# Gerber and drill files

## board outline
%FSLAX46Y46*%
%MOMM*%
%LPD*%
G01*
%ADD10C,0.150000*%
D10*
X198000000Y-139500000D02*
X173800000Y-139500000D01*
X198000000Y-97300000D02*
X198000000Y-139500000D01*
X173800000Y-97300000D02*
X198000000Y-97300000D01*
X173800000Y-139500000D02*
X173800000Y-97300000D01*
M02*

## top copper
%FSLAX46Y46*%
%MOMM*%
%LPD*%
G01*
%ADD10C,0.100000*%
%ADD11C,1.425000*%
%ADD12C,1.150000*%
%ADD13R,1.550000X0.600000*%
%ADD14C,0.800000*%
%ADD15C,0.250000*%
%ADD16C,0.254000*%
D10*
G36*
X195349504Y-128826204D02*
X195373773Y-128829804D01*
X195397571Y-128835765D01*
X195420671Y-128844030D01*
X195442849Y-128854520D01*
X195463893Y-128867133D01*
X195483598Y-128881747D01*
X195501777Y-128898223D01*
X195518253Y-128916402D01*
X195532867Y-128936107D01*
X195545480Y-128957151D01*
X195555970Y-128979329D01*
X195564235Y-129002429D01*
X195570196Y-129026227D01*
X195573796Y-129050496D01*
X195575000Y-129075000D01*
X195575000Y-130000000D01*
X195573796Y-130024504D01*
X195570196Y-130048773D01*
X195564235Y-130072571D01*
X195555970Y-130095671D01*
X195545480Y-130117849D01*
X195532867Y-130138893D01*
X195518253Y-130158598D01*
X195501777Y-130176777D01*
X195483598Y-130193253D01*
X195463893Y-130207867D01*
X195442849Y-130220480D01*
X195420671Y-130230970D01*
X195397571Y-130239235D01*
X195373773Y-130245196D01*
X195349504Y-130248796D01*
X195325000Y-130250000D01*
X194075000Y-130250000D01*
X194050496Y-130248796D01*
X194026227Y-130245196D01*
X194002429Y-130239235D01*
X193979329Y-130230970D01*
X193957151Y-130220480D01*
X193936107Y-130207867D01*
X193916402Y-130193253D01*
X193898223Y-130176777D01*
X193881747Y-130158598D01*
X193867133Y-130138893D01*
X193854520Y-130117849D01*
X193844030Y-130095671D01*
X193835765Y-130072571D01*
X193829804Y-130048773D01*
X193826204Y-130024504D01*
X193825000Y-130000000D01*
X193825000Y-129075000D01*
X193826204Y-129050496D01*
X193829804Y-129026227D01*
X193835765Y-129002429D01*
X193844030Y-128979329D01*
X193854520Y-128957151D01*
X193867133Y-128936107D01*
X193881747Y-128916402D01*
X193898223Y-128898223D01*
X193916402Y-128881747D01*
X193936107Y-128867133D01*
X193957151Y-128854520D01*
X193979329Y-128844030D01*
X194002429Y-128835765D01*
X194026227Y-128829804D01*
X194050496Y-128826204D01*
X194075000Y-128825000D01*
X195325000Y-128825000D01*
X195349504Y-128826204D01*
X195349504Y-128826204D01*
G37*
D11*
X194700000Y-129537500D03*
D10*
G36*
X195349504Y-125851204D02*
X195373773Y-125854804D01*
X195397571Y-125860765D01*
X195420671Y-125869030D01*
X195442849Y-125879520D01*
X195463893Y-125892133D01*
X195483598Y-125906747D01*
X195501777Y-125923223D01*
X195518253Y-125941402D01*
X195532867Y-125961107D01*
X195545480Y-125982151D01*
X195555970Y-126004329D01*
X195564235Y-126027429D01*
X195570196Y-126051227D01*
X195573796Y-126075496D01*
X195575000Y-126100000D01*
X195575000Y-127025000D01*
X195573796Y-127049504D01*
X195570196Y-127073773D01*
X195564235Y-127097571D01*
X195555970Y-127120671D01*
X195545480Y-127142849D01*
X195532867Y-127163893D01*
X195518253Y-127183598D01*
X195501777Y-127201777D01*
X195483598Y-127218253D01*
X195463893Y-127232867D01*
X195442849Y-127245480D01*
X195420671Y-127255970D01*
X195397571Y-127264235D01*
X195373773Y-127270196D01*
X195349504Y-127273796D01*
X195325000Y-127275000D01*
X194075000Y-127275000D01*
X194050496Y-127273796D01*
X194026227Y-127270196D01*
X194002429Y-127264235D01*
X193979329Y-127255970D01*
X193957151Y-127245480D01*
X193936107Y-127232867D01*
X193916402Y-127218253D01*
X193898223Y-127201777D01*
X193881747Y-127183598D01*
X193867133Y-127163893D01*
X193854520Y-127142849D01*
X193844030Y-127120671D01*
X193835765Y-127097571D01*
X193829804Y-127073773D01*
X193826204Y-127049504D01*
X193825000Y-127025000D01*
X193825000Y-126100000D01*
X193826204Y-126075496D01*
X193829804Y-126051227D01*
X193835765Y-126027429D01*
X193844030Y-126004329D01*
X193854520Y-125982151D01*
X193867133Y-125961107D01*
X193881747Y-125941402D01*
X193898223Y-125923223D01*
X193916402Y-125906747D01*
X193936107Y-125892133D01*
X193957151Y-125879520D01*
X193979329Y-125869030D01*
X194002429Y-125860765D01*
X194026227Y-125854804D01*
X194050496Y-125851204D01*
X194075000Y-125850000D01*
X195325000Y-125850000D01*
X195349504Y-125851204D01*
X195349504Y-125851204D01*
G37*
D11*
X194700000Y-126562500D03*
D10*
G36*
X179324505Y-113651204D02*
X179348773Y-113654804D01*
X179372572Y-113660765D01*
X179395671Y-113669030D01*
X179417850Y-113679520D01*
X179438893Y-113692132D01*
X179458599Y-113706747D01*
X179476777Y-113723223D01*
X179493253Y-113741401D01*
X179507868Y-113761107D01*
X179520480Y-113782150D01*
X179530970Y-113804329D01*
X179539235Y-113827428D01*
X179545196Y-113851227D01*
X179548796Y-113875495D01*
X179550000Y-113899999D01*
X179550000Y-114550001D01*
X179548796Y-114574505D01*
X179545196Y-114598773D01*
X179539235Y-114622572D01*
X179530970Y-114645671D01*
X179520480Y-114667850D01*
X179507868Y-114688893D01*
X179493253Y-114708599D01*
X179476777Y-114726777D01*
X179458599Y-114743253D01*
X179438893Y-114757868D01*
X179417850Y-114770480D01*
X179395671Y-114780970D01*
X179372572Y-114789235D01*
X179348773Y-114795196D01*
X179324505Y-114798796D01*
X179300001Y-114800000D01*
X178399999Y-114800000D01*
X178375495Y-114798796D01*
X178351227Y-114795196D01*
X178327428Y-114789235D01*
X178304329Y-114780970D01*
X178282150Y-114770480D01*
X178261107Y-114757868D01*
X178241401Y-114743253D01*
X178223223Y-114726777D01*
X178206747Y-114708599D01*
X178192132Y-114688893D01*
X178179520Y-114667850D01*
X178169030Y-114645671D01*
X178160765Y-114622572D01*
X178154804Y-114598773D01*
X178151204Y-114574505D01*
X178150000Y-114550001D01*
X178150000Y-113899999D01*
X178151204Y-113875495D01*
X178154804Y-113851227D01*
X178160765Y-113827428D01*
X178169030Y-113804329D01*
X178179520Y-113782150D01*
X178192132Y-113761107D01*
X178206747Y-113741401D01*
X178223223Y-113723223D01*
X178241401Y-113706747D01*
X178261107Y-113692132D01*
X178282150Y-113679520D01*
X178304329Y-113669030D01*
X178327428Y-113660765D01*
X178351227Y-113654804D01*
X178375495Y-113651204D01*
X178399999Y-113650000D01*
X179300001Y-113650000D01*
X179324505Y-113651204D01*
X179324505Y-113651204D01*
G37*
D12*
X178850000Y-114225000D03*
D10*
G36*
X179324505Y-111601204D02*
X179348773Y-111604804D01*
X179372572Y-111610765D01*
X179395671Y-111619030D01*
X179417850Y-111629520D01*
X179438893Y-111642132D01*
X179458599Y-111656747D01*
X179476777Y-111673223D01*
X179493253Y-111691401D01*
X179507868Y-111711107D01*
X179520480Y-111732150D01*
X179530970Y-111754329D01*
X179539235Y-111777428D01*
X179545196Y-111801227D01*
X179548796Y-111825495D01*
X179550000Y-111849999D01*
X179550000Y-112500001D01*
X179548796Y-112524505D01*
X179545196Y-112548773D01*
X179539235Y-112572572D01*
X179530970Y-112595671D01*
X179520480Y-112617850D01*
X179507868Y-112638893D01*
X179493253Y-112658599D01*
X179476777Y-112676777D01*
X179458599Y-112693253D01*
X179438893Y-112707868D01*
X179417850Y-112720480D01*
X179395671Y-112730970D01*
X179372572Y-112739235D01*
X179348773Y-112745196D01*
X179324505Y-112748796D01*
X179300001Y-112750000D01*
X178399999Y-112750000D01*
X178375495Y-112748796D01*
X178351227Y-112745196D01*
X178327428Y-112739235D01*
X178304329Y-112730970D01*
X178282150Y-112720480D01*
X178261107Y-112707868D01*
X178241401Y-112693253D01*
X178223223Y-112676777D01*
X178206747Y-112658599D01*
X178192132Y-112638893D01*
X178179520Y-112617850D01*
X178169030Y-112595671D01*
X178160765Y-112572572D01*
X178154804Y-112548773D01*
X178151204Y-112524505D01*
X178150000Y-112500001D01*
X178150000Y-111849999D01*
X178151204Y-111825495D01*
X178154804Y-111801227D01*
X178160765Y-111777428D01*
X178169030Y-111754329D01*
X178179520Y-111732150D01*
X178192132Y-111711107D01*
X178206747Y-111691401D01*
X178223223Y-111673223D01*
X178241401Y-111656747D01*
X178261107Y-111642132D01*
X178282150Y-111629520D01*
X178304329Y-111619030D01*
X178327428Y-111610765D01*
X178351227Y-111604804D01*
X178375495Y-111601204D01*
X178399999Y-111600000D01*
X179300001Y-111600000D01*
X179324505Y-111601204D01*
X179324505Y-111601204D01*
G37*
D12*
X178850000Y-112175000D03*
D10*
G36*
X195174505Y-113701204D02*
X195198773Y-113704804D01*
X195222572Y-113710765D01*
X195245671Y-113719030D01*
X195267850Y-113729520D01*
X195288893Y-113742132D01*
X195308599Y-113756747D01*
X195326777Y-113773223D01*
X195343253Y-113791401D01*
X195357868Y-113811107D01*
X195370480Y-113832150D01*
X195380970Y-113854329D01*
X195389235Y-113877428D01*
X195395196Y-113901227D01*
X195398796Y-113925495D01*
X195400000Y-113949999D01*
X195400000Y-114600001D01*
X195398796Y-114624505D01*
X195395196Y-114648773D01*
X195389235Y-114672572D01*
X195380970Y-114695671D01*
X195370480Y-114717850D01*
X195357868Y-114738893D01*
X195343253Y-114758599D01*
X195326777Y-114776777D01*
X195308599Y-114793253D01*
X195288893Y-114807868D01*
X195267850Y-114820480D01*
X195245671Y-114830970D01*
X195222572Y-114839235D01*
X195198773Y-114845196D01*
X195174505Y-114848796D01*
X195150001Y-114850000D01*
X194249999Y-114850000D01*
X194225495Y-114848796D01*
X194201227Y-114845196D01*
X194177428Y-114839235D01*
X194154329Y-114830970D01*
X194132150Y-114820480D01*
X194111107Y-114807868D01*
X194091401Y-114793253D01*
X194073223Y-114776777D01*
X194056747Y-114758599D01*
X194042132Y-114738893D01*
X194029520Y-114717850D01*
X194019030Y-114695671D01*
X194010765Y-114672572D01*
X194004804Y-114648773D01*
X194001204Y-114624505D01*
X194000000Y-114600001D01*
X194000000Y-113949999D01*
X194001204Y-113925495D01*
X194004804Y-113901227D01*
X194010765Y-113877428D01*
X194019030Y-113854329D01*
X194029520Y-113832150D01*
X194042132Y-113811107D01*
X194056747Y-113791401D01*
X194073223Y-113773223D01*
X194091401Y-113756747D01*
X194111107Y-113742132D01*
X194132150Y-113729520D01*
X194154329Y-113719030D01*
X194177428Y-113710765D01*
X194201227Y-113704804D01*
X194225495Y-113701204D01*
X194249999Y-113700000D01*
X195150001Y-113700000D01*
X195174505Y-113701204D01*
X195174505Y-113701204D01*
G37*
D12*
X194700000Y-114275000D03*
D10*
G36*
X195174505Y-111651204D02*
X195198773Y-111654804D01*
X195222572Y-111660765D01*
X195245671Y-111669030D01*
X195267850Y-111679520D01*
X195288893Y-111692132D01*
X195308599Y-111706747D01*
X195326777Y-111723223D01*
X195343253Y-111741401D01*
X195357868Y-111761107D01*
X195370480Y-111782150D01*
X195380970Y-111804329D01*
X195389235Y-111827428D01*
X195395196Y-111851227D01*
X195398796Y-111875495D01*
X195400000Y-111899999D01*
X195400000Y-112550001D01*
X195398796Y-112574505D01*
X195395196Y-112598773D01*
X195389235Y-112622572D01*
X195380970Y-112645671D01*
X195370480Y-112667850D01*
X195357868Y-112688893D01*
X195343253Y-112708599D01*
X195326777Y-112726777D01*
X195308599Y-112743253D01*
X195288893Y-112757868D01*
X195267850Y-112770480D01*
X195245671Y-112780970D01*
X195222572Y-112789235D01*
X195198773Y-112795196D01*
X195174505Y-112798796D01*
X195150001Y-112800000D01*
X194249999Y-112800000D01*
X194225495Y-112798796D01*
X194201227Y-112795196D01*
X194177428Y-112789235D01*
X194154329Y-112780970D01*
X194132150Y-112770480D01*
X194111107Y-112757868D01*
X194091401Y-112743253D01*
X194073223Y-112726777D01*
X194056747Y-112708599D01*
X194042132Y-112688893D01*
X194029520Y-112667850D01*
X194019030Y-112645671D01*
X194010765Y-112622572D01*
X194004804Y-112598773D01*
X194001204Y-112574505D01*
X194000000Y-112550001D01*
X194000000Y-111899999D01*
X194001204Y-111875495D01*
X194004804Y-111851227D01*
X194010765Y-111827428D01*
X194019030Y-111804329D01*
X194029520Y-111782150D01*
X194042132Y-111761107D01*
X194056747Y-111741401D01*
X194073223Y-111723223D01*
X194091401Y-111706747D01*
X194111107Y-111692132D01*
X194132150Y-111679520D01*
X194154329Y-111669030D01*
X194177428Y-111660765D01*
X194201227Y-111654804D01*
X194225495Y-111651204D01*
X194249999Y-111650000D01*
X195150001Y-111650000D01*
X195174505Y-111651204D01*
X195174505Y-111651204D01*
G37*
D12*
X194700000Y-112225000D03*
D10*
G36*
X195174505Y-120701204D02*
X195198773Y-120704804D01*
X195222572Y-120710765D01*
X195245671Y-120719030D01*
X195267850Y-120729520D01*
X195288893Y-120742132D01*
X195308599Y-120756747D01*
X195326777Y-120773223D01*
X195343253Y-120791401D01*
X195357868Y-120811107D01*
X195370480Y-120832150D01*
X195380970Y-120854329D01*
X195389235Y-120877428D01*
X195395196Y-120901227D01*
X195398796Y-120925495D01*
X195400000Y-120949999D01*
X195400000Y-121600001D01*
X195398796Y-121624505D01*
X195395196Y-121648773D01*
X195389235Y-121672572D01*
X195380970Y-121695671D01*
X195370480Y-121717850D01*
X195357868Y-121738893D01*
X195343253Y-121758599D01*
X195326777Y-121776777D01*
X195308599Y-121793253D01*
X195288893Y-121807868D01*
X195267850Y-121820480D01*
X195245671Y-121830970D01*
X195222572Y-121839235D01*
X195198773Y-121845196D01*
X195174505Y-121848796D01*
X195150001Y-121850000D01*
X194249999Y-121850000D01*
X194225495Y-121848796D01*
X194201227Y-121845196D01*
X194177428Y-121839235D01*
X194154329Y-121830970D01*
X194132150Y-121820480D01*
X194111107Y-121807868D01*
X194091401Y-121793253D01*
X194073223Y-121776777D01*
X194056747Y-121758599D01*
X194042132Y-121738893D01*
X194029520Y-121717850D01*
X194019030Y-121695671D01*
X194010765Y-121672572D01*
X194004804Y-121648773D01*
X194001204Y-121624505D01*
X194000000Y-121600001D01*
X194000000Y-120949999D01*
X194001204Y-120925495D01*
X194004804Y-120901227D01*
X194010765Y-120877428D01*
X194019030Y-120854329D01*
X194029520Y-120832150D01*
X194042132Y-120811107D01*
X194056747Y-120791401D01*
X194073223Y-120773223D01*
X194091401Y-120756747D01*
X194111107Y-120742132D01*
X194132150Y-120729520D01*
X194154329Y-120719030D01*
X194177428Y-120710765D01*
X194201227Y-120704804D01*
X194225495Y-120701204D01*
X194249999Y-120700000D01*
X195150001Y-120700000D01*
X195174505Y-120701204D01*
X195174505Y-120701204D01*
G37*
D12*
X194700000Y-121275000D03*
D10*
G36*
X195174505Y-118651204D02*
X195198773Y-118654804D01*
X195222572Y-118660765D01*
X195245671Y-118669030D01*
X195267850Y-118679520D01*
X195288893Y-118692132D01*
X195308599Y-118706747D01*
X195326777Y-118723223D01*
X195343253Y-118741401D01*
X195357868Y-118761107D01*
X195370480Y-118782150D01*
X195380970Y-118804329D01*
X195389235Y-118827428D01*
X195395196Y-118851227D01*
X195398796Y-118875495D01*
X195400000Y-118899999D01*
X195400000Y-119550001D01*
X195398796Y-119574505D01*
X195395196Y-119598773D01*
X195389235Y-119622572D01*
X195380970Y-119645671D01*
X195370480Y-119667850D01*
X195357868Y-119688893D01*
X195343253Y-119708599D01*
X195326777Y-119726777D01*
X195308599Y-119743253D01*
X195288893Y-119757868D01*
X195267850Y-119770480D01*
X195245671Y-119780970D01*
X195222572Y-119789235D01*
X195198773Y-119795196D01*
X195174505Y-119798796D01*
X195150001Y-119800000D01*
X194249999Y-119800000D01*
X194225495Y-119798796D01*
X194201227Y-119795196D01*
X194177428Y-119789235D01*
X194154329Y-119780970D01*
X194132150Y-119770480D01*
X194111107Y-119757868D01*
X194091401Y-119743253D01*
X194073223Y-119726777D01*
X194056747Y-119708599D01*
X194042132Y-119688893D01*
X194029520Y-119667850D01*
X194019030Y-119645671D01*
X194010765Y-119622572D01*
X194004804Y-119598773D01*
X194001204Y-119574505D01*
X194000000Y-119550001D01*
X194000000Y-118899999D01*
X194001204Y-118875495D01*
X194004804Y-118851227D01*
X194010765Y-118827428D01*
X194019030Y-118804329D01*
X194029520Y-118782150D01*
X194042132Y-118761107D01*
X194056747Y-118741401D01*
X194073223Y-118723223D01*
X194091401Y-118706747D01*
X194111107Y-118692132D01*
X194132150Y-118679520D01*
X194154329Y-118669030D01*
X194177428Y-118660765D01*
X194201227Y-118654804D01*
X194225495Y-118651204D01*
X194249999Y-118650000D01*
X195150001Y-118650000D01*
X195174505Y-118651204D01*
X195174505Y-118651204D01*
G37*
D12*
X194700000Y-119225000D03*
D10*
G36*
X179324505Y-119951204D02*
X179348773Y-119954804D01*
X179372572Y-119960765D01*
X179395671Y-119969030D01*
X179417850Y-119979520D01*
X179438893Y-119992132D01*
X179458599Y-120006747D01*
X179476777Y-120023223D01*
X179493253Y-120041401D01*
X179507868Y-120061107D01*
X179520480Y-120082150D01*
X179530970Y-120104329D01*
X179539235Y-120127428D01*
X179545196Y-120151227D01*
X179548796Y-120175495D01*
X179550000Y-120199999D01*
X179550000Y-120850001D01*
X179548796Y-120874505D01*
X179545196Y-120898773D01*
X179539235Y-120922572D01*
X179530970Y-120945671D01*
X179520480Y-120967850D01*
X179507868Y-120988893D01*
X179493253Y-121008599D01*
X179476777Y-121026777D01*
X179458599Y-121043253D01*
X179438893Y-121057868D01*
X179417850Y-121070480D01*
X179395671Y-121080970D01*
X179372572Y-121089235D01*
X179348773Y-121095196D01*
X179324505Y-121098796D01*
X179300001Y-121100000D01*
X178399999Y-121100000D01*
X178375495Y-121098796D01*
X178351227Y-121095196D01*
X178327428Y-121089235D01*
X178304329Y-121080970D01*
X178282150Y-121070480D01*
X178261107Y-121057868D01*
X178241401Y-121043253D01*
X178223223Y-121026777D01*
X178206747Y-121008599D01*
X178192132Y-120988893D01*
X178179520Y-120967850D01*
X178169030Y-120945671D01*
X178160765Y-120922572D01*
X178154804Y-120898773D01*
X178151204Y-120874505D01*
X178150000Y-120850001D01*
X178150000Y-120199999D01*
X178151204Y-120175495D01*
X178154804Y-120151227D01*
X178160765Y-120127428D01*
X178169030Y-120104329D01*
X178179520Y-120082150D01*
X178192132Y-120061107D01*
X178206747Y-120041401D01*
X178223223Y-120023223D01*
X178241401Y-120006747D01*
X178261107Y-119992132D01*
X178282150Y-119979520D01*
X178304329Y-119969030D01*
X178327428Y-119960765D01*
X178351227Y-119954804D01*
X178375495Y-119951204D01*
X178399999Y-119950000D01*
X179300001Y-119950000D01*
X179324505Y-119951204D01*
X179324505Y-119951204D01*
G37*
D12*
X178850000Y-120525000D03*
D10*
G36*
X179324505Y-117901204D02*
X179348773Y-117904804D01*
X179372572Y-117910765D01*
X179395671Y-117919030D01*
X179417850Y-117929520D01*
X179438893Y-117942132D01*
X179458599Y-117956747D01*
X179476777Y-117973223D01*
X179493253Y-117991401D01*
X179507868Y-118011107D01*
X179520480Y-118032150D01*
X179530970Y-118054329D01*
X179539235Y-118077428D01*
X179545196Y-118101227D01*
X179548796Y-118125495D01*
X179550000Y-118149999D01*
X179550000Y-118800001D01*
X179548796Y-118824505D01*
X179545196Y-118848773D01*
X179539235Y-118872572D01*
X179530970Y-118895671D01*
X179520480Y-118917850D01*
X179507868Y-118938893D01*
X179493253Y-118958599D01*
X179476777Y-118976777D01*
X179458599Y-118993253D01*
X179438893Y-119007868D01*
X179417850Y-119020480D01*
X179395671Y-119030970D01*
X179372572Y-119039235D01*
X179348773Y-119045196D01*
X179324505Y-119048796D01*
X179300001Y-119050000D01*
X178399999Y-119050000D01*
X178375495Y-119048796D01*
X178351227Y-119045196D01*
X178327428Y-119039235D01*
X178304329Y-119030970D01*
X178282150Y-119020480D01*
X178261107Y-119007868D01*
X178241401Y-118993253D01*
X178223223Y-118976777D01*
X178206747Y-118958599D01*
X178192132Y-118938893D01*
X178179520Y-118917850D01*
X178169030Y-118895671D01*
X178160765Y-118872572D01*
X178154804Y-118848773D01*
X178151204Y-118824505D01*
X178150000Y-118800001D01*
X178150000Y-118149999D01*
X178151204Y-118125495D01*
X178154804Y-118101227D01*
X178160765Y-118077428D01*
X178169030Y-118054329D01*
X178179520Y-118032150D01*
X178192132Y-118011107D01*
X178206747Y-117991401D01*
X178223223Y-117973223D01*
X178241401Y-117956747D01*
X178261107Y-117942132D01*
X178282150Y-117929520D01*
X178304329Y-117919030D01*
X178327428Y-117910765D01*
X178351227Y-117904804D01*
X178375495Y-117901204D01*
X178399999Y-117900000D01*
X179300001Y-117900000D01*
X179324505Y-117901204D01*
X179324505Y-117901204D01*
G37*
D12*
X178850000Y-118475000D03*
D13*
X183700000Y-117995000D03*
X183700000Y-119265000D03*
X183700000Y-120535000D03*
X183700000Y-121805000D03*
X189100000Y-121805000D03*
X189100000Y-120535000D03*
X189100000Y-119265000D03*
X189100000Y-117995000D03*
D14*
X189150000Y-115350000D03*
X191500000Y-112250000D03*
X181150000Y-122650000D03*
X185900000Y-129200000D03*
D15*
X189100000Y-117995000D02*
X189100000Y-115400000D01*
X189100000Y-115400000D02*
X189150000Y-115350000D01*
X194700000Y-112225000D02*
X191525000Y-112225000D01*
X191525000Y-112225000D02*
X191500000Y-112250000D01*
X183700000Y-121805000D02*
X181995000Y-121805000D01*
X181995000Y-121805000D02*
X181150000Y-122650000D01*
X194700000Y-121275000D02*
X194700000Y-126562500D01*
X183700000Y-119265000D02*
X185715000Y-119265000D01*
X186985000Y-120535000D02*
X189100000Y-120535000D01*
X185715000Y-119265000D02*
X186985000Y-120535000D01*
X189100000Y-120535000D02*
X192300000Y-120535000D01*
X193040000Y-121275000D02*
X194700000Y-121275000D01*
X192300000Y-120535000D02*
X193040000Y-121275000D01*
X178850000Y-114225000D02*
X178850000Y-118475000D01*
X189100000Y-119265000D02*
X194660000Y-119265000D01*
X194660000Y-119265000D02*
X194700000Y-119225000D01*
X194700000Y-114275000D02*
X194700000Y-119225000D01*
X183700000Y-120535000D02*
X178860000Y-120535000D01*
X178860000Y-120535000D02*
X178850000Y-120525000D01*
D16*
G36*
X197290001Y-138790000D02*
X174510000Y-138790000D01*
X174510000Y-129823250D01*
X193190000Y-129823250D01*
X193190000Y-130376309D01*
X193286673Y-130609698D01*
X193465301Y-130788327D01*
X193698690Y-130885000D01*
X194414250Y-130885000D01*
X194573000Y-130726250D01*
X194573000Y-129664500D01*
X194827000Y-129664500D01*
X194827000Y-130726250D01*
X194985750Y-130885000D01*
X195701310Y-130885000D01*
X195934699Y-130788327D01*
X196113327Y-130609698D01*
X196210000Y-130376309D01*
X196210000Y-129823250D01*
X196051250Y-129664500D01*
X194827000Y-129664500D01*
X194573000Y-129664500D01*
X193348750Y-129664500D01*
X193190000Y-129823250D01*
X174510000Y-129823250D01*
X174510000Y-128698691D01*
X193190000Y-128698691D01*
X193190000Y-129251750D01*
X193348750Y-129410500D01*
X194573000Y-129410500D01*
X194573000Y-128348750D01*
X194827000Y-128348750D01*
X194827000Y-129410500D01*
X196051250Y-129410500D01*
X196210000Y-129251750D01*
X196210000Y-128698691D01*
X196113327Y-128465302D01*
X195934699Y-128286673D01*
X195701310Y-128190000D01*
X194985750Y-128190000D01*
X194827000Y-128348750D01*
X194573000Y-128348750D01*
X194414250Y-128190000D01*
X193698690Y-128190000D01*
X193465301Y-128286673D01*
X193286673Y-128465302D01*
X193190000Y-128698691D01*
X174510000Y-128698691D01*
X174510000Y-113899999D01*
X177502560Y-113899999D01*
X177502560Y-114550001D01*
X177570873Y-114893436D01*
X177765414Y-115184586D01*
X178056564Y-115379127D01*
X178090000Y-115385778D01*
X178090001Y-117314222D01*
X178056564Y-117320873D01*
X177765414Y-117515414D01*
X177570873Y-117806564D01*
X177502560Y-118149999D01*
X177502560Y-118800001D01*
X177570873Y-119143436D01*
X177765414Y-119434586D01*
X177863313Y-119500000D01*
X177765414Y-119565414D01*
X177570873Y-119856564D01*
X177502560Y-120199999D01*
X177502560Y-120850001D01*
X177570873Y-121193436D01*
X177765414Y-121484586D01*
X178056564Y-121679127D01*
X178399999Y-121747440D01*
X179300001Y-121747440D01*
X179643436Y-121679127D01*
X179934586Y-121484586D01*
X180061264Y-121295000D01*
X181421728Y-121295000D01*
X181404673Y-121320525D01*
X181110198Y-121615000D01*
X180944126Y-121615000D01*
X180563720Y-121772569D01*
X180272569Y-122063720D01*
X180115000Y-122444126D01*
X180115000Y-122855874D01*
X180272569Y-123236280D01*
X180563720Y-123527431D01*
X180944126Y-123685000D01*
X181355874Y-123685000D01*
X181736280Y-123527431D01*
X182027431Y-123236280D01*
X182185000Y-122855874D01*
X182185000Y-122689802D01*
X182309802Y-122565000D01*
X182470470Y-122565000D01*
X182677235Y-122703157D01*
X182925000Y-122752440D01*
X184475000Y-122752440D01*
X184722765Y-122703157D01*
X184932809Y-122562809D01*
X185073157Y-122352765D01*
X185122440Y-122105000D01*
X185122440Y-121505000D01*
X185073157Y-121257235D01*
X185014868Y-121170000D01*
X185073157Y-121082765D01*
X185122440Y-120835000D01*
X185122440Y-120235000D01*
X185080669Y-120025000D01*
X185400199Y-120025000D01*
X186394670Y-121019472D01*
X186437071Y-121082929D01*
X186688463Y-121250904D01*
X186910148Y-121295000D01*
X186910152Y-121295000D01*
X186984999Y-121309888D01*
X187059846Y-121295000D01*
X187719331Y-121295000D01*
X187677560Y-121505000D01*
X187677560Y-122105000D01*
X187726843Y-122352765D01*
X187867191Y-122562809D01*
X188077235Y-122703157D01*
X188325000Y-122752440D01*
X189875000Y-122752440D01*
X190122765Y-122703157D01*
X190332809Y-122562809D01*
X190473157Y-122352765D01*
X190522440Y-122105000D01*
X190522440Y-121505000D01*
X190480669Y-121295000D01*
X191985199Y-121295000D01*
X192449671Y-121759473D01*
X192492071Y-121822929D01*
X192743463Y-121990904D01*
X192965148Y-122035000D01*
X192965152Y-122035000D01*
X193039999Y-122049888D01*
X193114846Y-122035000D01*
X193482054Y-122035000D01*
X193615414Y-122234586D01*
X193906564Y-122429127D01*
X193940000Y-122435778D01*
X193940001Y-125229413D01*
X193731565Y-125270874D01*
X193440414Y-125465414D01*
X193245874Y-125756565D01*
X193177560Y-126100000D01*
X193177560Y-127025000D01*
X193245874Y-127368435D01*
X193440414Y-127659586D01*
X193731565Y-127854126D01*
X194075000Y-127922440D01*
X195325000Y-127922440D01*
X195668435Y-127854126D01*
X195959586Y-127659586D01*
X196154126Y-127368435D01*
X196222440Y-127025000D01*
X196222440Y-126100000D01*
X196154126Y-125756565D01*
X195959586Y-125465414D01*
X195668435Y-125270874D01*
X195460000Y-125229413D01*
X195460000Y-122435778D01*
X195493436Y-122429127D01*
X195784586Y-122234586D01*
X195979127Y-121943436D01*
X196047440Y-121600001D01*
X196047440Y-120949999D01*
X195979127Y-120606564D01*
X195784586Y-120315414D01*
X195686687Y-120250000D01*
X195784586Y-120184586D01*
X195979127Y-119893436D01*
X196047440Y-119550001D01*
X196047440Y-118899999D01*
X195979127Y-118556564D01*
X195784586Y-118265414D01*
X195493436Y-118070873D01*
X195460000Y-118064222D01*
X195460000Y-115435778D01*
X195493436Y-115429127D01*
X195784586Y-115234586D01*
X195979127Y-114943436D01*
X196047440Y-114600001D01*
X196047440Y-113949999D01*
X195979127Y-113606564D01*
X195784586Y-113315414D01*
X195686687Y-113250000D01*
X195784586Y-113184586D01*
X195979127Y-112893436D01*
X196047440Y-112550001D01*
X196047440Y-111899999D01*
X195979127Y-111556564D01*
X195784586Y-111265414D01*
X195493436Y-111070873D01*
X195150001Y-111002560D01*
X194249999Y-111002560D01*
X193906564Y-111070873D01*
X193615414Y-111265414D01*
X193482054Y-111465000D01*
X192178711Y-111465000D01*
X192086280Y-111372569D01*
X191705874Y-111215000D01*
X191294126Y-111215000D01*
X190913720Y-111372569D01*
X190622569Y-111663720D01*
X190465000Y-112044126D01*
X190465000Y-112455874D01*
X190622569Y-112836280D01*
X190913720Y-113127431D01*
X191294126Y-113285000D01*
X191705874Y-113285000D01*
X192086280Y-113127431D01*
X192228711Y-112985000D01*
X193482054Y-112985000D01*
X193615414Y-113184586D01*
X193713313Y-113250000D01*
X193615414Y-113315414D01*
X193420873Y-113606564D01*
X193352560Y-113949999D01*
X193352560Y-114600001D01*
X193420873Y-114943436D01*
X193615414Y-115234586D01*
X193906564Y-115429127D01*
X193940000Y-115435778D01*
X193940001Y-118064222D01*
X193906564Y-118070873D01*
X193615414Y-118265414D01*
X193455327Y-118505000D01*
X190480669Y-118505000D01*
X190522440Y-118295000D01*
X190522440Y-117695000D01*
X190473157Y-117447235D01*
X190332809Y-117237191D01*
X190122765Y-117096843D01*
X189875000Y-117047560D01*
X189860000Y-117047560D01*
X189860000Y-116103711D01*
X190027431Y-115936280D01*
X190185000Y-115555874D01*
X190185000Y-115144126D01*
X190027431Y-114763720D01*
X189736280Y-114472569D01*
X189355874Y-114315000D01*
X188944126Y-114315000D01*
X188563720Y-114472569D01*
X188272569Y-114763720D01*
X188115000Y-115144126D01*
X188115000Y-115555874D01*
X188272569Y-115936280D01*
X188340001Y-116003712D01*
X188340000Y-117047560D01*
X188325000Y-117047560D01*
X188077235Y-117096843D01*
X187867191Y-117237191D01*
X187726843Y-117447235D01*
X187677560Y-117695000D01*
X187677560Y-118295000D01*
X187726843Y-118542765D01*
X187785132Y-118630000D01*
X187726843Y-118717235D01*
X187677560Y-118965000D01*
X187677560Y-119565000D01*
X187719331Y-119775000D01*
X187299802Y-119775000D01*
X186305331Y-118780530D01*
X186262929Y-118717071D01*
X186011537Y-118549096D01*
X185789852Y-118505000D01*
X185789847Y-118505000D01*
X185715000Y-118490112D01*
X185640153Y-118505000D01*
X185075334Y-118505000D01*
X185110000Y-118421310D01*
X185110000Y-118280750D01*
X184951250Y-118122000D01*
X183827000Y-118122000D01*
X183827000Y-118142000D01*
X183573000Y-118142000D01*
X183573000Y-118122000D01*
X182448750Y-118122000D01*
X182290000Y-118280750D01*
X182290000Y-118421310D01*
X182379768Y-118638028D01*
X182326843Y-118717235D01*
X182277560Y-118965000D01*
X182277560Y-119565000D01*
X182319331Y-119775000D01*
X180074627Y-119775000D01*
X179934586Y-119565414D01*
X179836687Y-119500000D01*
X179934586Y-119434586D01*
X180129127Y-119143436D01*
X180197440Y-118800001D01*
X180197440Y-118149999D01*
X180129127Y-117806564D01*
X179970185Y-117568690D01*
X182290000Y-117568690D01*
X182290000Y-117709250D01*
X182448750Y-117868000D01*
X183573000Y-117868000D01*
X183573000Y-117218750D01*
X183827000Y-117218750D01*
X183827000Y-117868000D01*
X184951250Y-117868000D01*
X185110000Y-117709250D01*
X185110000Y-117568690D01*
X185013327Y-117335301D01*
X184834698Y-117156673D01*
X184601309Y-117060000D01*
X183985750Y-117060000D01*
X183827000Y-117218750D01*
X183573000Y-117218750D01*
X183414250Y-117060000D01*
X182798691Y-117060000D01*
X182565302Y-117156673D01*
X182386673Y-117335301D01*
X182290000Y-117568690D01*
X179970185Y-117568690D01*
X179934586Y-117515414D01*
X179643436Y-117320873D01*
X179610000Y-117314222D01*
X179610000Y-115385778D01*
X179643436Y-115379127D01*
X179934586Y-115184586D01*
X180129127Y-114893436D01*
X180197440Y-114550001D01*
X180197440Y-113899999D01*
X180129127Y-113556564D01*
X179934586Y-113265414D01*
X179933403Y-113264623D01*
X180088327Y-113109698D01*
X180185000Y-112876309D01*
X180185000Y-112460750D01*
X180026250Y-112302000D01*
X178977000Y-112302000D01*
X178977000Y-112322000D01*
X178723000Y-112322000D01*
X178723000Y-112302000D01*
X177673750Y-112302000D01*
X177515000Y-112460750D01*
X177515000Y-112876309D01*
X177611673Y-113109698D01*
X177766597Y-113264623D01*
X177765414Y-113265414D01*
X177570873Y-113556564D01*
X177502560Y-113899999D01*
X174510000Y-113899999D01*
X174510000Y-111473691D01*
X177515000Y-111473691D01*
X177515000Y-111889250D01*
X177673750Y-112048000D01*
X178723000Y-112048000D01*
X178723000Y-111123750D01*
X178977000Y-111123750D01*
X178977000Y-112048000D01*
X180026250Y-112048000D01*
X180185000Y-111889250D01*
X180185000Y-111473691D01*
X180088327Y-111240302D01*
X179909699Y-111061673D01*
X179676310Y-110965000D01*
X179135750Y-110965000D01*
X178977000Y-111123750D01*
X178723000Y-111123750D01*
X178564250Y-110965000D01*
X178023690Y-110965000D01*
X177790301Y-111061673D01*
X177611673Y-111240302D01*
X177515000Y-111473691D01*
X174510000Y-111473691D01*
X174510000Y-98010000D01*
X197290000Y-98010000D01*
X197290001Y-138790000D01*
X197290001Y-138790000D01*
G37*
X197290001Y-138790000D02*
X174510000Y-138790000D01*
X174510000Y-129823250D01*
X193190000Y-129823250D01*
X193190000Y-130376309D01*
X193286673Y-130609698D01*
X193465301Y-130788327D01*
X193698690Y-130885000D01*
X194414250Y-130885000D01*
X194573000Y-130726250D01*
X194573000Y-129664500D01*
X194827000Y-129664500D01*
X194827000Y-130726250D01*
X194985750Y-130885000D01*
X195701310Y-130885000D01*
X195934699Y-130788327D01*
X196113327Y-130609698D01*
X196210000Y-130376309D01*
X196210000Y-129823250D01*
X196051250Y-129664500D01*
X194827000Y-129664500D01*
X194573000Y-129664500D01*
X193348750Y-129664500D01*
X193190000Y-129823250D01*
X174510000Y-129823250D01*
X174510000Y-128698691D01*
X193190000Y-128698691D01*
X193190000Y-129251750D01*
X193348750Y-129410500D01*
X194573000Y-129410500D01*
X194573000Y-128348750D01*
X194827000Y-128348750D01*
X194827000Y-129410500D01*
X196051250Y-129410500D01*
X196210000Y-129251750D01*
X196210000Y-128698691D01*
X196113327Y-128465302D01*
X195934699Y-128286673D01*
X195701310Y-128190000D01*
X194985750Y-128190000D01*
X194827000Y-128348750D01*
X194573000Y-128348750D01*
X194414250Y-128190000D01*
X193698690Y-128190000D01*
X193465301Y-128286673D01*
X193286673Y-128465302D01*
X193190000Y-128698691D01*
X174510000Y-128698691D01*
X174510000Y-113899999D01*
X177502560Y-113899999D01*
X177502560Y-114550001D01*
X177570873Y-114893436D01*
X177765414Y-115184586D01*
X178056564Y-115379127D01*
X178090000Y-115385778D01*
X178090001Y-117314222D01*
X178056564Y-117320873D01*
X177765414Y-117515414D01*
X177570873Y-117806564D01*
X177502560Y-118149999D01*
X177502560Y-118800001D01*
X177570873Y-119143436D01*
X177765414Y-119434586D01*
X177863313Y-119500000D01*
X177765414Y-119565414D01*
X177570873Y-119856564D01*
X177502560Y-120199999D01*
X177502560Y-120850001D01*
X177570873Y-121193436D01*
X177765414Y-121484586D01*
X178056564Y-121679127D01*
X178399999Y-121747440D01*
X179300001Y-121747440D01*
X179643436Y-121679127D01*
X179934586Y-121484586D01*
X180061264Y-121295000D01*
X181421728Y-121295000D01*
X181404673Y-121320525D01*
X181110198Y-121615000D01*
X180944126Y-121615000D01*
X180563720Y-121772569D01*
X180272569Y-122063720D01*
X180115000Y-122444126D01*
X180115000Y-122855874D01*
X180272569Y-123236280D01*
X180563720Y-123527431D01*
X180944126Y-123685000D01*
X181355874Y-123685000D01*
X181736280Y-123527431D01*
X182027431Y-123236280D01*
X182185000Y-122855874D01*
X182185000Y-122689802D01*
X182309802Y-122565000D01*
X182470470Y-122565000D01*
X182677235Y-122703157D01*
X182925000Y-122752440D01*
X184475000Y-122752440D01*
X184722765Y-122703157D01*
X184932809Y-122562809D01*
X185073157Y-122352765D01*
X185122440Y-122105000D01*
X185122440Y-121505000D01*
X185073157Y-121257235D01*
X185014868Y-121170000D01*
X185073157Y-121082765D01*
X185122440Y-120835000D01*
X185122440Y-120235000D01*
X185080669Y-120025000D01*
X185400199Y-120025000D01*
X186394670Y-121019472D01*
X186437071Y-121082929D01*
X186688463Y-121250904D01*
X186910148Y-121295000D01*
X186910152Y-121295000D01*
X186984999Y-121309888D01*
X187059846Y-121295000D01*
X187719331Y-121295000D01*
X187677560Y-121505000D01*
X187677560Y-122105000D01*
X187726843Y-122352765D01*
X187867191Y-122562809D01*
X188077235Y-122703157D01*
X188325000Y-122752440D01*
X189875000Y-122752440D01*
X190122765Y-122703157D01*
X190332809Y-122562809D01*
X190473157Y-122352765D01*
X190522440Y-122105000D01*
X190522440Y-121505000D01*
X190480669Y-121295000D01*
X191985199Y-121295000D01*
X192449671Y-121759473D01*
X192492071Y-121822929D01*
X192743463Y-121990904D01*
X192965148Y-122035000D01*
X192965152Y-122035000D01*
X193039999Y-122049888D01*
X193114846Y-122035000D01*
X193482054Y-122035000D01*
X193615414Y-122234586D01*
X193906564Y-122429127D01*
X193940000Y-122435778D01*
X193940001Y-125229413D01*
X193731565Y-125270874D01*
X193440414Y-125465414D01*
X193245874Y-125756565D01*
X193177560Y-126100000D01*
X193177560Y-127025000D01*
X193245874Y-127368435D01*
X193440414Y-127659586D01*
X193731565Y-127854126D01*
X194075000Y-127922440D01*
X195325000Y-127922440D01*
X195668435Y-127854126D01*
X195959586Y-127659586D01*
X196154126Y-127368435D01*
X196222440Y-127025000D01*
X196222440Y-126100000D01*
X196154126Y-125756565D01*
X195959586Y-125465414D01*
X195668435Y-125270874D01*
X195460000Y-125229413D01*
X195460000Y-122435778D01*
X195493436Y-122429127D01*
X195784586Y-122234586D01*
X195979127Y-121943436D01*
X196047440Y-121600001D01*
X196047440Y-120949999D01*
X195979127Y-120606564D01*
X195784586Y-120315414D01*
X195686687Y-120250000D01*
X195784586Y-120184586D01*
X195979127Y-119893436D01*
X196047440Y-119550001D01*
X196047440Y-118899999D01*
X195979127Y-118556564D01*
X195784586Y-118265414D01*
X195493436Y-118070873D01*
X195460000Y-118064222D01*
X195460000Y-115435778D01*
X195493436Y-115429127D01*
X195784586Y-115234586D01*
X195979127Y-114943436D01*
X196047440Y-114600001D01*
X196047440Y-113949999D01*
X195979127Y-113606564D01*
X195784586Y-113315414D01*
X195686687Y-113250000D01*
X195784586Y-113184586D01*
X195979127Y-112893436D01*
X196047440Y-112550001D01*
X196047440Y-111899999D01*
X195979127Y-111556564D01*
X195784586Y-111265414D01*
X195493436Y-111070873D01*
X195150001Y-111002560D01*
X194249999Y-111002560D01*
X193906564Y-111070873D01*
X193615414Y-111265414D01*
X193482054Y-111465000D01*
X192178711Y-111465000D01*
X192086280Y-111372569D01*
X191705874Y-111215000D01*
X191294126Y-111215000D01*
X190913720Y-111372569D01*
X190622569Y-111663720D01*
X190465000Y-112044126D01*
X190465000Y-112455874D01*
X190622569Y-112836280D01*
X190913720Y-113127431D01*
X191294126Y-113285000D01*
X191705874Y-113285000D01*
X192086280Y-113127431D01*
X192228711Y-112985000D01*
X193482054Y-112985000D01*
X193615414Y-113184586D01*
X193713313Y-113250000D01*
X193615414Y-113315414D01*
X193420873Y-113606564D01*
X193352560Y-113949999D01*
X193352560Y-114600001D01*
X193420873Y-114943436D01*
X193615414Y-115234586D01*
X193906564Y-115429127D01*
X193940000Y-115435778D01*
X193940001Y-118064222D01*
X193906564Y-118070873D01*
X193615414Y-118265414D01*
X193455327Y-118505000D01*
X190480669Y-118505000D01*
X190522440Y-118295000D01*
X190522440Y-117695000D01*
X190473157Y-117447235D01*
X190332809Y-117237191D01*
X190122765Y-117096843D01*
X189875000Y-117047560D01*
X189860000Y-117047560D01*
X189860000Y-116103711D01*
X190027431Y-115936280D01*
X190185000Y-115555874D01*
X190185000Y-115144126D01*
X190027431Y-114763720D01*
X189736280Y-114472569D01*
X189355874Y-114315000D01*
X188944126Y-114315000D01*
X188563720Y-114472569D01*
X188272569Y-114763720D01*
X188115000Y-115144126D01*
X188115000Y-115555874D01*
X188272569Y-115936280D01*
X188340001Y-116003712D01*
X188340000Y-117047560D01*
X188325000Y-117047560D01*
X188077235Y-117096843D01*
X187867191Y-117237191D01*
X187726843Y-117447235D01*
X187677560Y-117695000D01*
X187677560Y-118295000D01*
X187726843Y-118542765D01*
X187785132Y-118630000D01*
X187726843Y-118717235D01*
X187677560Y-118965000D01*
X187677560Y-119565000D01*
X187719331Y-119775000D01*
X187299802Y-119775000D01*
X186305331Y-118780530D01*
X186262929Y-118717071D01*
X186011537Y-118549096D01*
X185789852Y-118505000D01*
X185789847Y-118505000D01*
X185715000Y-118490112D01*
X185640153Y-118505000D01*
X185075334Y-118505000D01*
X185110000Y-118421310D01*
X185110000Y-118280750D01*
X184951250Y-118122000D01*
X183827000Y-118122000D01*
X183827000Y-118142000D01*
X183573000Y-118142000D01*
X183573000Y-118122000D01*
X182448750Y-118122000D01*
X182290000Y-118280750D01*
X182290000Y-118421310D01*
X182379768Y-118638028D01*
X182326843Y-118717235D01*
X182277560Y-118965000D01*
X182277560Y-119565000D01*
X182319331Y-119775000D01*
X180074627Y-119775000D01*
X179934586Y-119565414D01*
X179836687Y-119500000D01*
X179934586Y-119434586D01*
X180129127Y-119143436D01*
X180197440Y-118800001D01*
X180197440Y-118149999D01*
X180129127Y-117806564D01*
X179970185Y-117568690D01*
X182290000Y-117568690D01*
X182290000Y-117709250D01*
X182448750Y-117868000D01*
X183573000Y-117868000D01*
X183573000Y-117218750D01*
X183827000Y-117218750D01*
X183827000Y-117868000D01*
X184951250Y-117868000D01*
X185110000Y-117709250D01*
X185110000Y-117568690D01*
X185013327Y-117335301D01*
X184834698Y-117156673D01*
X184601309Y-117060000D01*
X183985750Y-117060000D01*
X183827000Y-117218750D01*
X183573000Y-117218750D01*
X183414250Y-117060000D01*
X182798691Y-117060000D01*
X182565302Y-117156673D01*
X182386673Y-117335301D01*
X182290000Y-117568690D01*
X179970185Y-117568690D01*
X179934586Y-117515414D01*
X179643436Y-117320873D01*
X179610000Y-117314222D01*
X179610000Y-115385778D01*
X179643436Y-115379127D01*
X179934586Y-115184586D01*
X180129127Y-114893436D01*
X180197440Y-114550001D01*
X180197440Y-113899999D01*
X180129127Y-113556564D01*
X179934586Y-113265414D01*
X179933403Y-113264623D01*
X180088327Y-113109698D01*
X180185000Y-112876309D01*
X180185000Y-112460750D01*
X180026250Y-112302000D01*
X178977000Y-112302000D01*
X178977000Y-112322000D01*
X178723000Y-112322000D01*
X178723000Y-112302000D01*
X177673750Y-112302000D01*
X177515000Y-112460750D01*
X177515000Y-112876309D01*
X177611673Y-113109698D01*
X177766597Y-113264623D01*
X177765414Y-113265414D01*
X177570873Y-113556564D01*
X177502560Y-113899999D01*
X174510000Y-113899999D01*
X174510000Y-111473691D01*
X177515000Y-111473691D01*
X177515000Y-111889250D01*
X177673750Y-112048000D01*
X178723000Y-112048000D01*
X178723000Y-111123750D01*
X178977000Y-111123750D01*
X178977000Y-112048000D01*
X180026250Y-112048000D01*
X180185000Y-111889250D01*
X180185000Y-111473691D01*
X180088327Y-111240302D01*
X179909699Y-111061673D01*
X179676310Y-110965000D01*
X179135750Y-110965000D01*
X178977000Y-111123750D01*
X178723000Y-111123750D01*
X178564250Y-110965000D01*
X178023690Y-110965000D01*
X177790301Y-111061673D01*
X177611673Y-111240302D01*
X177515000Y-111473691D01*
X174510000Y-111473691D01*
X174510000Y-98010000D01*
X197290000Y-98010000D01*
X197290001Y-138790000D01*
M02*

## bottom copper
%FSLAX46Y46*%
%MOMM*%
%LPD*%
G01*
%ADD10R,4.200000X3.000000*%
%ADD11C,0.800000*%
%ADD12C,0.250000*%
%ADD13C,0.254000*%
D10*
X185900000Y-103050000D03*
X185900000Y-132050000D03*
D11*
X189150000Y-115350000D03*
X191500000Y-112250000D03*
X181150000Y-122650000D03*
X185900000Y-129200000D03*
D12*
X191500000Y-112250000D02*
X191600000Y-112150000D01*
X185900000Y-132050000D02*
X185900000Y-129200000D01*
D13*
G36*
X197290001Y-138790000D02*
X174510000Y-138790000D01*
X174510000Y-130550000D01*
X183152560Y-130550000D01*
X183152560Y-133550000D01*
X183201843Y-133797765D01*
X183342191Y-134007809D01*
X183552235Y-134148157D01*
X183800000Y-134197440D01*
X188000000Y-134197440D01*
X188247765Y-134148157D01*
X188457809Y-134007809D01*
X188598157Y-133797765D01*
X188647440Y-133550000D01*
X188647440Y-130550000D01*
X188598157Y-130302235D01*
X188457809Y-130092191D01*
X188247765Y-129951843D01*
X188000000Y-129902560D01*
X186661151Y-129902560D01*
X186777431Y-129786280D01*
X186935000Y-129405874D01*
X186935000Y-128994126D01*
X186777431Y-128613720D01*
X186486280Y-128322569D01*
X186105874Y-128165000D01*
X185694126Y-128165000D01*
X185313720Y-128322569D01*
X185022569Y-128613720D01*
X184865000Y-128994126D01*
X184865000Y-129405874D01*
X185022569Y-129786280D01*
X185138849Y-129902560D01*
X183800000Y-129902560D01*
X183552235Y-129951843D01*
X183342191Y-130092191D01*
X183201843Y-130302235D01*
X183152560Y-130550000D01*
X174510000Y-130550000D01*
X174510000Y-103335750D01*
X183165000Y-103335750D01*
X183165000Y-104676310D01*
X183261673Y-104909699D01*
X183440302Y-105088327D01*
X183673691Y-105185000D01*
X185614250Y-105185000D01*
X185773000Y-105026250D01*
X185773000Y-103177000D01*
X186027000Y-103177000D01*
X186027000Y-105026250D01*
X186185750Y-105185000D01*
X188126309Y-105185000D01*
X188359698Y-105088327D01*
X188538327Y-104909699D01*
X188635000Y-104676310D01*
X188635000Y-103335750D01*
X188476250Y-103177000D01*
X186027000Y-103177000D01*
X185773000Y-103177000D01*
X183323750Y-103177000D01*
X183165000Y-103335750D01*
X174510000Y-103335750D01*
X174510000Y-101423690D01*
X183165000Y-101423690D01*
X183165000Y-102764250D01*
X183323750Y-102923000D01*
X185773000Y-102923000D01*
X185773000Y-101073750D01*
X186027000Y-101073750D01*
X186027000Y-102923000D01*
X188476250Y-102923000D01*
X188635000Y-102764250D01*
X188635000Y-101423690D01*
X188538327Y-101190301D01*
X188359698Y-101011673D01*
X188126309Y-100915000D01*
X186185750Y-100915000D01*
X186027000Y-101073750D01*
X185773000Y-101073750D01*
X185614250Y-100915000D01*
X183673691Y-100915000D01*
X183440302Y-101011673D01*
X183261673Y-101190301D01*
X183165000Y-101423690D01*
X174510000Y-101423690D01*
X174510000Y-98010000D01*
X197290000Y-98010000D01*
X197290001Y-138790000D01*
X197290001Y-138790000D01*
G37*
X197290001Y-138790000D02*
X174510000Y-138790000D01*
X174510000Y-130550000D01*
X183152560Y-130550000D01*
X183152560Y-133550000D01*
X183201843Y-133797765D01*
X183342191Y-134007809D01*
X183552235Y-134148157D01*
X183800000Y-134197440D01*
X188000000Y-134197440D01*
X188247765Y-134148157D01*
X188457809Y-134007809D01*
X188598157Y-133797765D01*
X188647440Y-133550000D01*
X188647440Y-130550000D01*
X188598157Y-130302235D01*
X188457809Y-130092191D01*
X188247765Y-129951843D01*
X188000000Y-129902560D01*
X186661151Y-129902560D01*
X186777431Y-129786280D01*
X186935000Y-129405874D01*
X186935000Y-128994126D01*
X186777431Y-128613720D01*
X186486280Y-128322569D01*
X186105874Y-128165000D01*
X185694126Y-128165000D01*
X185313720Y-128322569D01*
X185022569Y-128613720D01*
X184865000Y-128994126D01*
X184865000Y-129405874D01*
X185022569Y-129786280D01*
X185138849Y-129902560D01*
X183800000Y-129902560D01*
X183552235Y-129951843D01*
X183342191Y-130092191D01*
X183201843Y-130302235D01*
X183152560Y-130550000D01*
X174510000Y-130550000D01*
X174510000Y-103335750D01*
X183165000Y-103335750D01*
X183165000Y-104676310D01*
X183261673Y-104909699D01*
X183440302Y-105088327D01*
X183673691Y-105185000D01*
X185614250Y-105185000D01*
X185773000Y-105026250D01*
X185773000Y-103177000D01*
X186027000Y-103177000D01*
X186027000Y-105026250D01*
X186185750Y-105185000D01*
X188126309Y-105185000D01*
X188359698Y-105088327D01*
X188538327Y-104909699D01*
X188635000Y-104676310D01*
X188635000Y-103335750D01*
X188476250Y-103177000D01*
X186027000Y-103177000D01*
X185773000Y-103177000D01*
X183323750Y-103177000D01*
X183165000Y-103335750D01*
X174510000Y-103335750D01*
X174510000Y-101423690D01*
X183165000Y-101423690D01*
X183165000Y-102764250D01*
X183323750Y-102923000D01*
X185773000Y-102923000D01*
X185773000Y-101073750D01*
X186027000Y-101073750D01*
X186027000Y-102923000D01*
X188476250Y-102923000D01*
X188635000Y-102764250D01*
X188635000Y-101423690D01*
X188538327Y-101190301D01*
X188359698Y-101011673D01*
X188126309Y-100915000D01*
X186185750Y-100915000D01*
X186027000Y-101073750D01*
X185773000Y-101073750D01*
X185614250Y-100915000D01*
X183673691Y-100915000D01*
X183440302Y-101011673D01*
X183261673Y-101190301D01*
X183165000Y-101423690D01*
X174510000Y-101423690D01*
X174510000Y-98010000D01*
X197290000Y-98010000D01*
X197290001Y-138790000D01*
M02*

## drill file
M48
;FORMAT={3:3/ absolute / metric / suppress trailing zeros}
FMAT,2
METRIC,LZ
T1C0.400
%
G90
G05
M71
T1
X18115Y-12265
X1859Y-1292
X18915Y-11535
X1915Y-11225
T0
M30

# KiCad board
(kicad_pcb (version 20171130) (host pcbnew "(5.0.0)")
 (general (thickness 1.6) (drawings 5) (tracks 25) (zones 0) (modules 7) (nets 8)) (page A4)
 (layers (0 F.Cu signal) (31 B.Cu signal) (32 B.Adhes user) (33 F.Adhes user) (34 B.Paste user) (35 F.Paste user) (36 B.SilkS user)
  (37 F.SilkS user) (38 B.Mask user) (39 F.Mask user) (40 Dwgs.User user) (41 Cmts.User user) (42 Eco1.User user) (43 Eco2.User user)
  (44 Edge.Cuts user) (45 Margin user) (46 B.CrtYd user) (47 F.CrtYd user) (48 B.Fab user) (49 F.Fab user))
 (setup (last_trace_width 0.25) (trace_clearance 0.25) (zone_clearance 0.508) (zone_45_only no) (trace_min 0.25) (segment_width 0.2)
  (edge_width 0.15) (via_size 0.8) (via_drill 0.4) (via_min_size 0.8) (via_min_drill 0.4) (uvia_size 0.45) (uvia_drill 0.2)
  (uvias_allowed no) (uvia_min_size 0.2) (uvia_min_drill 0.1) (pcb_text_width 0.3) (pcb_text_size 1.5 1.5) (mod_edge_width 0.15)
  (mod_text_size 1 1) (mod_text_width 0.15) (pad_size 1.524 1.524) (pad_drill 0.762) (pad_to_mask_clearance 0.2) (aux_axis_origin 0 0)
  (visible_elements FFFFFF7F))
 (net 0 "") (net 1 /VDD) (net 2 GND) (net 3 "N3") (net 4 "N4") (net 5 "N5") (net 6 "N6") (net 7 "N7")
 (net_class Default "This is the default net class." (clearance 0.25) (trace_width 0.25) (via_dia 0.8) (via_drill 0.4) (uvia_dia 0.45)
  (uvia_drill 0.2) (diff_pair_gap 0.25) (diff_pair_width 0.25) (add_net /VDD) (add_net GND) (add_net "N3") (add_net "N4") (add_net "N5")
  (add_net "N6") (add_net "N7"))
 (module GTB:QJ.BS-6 (layer B.Cu) (at 185.9 117.55 180)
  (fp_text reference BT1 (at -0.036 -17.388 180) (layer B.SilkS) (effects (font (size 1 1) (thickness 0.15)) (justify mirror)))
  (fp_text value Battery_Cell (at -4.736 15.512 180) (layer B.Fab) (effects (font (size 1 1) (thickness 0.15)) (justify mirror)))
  (pad 1 smd rect (at 0 14.5 180) (size 4.2 3) (layers B.Cu B.Paste B.Mask) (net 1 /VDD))
  (pad 2 smd rect (at 0 -14.5 180) (size 4.2 3) (layers B.Cu B.Paste B.Mask) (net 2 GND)))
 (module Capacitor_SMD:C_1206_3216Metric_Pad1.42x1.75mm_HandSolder (layer F.Cu) (at 194.7 128.05 270)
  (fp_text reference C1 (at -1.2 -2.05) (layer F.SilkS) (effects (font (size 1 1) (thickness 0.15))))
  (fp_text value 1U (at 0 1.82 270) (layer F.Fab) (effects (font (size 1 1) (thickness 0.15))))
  (pad 2 smd roundrect (at 1.4875 0 270) (size 1.425 1.75) (layers F.Cu F.Paste F.Mask) (roundrect_rratio 0.175439) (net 2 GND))
  (pad 1 smd roundrect (at -1.4875 0 270) (size 1.425 1.75) (layers F.Cu F.Paste F.Mask) (roundrect_rratio 0.175439) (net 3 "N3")))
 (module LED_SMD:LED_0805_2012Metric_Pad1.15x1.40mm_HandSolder (layer F.Cu) (at 178.85 113.2 270)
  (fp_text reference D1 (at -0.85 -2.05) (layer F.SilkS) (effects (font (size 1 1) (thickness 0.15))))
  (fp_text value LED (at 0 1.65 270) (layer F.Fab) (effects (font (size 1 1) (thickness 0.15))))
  (pad 2 smd roundrect (at 1.025 0 270) (size 1.15 1.4) (layers F.Cu F.Paste F.Mask) (roundrect_rratio 0.217391) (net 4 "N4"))
  (pad 1 smd roundrect (at -1.025 0 270) (size 1.15 1.4) (layers F.Cu F.Paste F.Mask) (roundrect_rratio 0.217391) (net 2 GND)))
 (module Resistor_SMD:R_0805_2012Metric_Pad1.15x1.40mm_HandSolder (layer F.Cu) (at 194.7 113.25 270)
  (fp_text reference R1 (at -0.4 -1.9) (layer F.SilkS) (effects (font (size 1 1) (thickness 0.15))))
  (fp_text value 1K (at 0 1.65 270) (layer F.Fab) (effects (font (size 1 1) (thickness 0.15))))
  (pad 2 smd roundrect (at 1.025 0 270) (size 1.15 1.4) (layers F.Cu F.Paste F.Mask) (roundrect_rratio 0.217391) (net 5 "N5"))
  (pad 1 smd roundrect (at -1.025 0 270) (size 1.15 1.4) (layers F.Cu F.Paste F.Mask) (roundrect_rratio 0.217391) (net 1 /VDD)))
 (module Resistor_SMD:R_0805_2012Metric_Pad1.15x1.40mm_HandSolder (layer F.Cu) (at 194.7 120.25 270)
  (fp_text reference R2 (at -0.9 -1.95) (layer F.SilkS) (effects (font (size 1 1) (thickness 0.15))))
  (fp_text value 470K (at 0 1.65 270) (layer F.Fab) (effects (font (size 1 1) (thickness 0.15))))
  (pad 2 smd roundrect (at 1.025 0 270) (size 1.15 1.4) (layers F.Cu F.Paste F.Mask) (roundrect_rratio 0.217391) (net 3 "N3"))
  (pad 1 smd roundrect (at -1.025 0 270) (size 1.15 1.4) (layers F.Cu F.Paste F.Mask) (roundrect_rratio 0.217391) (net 5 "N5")))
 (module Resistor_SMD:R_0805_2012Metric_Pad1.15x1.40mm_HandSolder (layer F.Cu) (at 178.85 119.5 90)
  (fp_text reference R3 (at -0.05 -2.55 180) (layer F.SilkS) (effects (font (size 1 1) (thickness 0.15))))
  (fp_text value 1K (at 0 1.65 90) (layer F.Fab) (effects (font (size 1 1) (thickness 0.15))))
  (pad 1 smd roundrect (at -1.025 0 90) (size 1.15 1.4) (layers F.Cu F.Paste F.Mask) (roundrect_rratio 0.217391) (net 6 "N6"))
  (pad 2 smd roundrect (at 1.025 0 90) (size 1.15 1.4) (layers F.Cu F.Paste F.Mask) (roundrect_rratio 0.217391) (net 4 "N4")))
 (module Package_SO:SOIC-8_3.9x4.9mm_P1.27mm (layer F.Cu) (at 186.4 119.9)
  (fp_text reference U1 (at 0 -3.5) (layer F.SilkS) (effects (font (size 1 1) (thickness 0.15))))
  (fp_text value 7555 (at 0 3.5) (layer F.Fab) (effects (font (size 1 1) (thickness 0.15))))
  (pad 1 smd rect (at -2.7 -1.905) (size 1.55 0.6) (layers F.Cu F.Paste F.Mask) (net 2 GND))
  (pad 2 smd rect (at -2.7 -0.635) (size 1.55 0.6) (layers F.Cu F.Paste F.Mask) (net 3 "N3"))
  (pad 3 smd rect (at -2.7 0.635) (size 1.55 0.6) (layers F.Cu F.Paste F.Mask) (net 6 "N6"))
  (pad 4 smd rect (at -2.7 1.905) (size 1.55 0.6) (layers F.Cu F.Paste F.Mask) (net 1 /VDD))
  (pad 5 smd rect (at 2.7 1.905) (size 1.55 0.6) (layers F.Cu F.Paste F.Mask) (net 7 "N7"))
  (pad 6 smd rect (at 2.7 0.635) (size 1.55 0.6) (layers F.Cu F.Paste F.Mask) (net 3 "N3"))
  (pad 7 smd rect (at 2.7 -0.635) (size 1.55 0.6) (layers F.Cu F.Paste F.Mask) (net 5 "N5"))
  (pad 8 smd rect (at 2.7 -1.905) (size 1.55 0.6) (layers F.Cu F.Paste F.Mask) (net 1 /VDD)))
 (gr_line (start 198 139.5) (end 173.8 139.5) (angle 90) (layer Edge.Cuts) (width 0.15))
 (gr_line (start 198 97.3) (end 198 139.5) (angle 90) (layer Edge.Cuts) (width 0.15))
 (gr_line (start 173.8 97.3) (end 198 97.3) (angle 90) (layer Edge.Cuts) (width 0.15))
 (gr_line (start 173.8 139.5) (end 173.8 97.3) (angle 90) (layer Edge.Cuts) (width 0.15))
 (segment (start 189.1 117.995) (end 189.1 115.4) (width 0.25) (layer F.Cu) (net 1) (status 400000))
 (via (at 189.15 115.35) (size 0.8) (drill 0.4) (layers F.Cu B.Cu) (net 1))
 (segment (start 189.1 115.4) (end 189.15 115.35) (width 0.25) (layer F.Cu) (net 1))
 (segment (start 194.7 112.225) (end 191.525 112.225) (width 0.25) (layer F.Cu) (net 1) (status 400000))
 (segment (start 191.5 112.25) (end 191.6 112.15) (width 0.25) (layer B.Cu) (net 1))
 (via (at 191.5 112.25) (size 0.8) (drill 0.4) (layers F.Cu B.Cu) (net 1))
 (segment (start 191.525 112.225) (end 191.5 112.25) (width 0.25) (layer F.Cu) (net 1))
 (segment (start 183.7 121.805) (end 181.995 121.805) (width 0.25) (layer F.Cu) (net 1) (status 400000))
 (via (at 181.15 122.65) (size 0.8) (drill 0.4) (layers F.Cu B.Cu) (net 1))
 (segment (start 181.995 121.805) (end 181.15 122.65) (width 0.25) (layer F.Cu) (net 1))
 (segment (start 185.9 132.05) (end 185.9 129.2) (width 0.25) (layer B.Cu) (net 2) (status 400000))
 (via (at 185.9 129.2) (size 0.8) (drill 0.4) (layers F.Cu B.Cu) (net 2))
 (segment (start 194.7 121.275) (end 194.7 126.5625) (width 0.25) (layer F.Cu) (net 3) (status C00000))
 (segment (start 183.7 119.265) (end 185.715 119.265) (width 0.25) (layer F.Cu) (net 3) (status 400000))
 (segment (start 186.985 120.535) (end 189.1 120.535) (width 0.25) (layer F.Cu) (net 3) (status 800000))
 (segment (start 185.715 119.265) (end 186.985 120.535) (width 0.25) (layer F.Cu) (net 3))
 (segment (start 189.1 120.535) (end 192.3 120.535) (width 0.25) (layer F.Cu) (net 3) (status 400000))
 (segment (start 193.04 121.275) (end 194.7 121.275) (width 0.25) (layer F.Cu) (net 3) (status 800000))
 (segment (start 192.3 120.535) (end 193.04 121.275) (width 0.25) (layer F.Cu) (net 3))
 (segment (start 178.85 114.225) (end 178.85 118.475) (width 0.25) (layer F.Cu) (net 4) (status C00000))
 (segment (start 189.1 119.265) (end 194.66 119.265) (width 0.25) (layer F.Cu) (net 5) (status C00000))
 (segment (start 194.66 119.265) (end 194.7 119.225) (width 0.25) (layer F.Cu) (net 5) (status C00000))
 (segment (start 194.7 114.275) (end 194.7 119.225) (width 0.25) (layer F.Cu) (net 5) (status C00000))
 (segment (start 183.7 120.535) (end 178.86 120.535) (width 0.25) (layer F.Cu) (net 6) (status C00000))
 (segment (start 178.86 120.535) (end 178.85 120.525) (width 0.25) (layer F.Cu) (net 6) (status C00000))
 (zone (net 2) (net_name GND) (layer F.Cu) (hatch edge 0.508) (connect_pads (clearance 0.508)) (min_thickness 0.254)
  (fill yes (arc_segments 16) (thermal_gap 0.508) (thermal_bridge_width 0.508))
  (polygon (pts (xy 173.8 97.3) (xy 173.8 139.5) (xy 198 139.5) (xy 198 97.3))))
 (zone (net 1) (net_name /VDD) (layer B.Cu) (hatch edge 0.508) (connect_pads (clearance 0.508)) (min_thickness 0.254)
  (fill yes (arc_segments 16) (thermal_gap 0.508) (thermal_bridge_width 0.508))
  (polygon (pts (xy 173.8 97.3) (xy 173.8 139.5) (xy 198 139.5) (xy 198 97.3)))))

